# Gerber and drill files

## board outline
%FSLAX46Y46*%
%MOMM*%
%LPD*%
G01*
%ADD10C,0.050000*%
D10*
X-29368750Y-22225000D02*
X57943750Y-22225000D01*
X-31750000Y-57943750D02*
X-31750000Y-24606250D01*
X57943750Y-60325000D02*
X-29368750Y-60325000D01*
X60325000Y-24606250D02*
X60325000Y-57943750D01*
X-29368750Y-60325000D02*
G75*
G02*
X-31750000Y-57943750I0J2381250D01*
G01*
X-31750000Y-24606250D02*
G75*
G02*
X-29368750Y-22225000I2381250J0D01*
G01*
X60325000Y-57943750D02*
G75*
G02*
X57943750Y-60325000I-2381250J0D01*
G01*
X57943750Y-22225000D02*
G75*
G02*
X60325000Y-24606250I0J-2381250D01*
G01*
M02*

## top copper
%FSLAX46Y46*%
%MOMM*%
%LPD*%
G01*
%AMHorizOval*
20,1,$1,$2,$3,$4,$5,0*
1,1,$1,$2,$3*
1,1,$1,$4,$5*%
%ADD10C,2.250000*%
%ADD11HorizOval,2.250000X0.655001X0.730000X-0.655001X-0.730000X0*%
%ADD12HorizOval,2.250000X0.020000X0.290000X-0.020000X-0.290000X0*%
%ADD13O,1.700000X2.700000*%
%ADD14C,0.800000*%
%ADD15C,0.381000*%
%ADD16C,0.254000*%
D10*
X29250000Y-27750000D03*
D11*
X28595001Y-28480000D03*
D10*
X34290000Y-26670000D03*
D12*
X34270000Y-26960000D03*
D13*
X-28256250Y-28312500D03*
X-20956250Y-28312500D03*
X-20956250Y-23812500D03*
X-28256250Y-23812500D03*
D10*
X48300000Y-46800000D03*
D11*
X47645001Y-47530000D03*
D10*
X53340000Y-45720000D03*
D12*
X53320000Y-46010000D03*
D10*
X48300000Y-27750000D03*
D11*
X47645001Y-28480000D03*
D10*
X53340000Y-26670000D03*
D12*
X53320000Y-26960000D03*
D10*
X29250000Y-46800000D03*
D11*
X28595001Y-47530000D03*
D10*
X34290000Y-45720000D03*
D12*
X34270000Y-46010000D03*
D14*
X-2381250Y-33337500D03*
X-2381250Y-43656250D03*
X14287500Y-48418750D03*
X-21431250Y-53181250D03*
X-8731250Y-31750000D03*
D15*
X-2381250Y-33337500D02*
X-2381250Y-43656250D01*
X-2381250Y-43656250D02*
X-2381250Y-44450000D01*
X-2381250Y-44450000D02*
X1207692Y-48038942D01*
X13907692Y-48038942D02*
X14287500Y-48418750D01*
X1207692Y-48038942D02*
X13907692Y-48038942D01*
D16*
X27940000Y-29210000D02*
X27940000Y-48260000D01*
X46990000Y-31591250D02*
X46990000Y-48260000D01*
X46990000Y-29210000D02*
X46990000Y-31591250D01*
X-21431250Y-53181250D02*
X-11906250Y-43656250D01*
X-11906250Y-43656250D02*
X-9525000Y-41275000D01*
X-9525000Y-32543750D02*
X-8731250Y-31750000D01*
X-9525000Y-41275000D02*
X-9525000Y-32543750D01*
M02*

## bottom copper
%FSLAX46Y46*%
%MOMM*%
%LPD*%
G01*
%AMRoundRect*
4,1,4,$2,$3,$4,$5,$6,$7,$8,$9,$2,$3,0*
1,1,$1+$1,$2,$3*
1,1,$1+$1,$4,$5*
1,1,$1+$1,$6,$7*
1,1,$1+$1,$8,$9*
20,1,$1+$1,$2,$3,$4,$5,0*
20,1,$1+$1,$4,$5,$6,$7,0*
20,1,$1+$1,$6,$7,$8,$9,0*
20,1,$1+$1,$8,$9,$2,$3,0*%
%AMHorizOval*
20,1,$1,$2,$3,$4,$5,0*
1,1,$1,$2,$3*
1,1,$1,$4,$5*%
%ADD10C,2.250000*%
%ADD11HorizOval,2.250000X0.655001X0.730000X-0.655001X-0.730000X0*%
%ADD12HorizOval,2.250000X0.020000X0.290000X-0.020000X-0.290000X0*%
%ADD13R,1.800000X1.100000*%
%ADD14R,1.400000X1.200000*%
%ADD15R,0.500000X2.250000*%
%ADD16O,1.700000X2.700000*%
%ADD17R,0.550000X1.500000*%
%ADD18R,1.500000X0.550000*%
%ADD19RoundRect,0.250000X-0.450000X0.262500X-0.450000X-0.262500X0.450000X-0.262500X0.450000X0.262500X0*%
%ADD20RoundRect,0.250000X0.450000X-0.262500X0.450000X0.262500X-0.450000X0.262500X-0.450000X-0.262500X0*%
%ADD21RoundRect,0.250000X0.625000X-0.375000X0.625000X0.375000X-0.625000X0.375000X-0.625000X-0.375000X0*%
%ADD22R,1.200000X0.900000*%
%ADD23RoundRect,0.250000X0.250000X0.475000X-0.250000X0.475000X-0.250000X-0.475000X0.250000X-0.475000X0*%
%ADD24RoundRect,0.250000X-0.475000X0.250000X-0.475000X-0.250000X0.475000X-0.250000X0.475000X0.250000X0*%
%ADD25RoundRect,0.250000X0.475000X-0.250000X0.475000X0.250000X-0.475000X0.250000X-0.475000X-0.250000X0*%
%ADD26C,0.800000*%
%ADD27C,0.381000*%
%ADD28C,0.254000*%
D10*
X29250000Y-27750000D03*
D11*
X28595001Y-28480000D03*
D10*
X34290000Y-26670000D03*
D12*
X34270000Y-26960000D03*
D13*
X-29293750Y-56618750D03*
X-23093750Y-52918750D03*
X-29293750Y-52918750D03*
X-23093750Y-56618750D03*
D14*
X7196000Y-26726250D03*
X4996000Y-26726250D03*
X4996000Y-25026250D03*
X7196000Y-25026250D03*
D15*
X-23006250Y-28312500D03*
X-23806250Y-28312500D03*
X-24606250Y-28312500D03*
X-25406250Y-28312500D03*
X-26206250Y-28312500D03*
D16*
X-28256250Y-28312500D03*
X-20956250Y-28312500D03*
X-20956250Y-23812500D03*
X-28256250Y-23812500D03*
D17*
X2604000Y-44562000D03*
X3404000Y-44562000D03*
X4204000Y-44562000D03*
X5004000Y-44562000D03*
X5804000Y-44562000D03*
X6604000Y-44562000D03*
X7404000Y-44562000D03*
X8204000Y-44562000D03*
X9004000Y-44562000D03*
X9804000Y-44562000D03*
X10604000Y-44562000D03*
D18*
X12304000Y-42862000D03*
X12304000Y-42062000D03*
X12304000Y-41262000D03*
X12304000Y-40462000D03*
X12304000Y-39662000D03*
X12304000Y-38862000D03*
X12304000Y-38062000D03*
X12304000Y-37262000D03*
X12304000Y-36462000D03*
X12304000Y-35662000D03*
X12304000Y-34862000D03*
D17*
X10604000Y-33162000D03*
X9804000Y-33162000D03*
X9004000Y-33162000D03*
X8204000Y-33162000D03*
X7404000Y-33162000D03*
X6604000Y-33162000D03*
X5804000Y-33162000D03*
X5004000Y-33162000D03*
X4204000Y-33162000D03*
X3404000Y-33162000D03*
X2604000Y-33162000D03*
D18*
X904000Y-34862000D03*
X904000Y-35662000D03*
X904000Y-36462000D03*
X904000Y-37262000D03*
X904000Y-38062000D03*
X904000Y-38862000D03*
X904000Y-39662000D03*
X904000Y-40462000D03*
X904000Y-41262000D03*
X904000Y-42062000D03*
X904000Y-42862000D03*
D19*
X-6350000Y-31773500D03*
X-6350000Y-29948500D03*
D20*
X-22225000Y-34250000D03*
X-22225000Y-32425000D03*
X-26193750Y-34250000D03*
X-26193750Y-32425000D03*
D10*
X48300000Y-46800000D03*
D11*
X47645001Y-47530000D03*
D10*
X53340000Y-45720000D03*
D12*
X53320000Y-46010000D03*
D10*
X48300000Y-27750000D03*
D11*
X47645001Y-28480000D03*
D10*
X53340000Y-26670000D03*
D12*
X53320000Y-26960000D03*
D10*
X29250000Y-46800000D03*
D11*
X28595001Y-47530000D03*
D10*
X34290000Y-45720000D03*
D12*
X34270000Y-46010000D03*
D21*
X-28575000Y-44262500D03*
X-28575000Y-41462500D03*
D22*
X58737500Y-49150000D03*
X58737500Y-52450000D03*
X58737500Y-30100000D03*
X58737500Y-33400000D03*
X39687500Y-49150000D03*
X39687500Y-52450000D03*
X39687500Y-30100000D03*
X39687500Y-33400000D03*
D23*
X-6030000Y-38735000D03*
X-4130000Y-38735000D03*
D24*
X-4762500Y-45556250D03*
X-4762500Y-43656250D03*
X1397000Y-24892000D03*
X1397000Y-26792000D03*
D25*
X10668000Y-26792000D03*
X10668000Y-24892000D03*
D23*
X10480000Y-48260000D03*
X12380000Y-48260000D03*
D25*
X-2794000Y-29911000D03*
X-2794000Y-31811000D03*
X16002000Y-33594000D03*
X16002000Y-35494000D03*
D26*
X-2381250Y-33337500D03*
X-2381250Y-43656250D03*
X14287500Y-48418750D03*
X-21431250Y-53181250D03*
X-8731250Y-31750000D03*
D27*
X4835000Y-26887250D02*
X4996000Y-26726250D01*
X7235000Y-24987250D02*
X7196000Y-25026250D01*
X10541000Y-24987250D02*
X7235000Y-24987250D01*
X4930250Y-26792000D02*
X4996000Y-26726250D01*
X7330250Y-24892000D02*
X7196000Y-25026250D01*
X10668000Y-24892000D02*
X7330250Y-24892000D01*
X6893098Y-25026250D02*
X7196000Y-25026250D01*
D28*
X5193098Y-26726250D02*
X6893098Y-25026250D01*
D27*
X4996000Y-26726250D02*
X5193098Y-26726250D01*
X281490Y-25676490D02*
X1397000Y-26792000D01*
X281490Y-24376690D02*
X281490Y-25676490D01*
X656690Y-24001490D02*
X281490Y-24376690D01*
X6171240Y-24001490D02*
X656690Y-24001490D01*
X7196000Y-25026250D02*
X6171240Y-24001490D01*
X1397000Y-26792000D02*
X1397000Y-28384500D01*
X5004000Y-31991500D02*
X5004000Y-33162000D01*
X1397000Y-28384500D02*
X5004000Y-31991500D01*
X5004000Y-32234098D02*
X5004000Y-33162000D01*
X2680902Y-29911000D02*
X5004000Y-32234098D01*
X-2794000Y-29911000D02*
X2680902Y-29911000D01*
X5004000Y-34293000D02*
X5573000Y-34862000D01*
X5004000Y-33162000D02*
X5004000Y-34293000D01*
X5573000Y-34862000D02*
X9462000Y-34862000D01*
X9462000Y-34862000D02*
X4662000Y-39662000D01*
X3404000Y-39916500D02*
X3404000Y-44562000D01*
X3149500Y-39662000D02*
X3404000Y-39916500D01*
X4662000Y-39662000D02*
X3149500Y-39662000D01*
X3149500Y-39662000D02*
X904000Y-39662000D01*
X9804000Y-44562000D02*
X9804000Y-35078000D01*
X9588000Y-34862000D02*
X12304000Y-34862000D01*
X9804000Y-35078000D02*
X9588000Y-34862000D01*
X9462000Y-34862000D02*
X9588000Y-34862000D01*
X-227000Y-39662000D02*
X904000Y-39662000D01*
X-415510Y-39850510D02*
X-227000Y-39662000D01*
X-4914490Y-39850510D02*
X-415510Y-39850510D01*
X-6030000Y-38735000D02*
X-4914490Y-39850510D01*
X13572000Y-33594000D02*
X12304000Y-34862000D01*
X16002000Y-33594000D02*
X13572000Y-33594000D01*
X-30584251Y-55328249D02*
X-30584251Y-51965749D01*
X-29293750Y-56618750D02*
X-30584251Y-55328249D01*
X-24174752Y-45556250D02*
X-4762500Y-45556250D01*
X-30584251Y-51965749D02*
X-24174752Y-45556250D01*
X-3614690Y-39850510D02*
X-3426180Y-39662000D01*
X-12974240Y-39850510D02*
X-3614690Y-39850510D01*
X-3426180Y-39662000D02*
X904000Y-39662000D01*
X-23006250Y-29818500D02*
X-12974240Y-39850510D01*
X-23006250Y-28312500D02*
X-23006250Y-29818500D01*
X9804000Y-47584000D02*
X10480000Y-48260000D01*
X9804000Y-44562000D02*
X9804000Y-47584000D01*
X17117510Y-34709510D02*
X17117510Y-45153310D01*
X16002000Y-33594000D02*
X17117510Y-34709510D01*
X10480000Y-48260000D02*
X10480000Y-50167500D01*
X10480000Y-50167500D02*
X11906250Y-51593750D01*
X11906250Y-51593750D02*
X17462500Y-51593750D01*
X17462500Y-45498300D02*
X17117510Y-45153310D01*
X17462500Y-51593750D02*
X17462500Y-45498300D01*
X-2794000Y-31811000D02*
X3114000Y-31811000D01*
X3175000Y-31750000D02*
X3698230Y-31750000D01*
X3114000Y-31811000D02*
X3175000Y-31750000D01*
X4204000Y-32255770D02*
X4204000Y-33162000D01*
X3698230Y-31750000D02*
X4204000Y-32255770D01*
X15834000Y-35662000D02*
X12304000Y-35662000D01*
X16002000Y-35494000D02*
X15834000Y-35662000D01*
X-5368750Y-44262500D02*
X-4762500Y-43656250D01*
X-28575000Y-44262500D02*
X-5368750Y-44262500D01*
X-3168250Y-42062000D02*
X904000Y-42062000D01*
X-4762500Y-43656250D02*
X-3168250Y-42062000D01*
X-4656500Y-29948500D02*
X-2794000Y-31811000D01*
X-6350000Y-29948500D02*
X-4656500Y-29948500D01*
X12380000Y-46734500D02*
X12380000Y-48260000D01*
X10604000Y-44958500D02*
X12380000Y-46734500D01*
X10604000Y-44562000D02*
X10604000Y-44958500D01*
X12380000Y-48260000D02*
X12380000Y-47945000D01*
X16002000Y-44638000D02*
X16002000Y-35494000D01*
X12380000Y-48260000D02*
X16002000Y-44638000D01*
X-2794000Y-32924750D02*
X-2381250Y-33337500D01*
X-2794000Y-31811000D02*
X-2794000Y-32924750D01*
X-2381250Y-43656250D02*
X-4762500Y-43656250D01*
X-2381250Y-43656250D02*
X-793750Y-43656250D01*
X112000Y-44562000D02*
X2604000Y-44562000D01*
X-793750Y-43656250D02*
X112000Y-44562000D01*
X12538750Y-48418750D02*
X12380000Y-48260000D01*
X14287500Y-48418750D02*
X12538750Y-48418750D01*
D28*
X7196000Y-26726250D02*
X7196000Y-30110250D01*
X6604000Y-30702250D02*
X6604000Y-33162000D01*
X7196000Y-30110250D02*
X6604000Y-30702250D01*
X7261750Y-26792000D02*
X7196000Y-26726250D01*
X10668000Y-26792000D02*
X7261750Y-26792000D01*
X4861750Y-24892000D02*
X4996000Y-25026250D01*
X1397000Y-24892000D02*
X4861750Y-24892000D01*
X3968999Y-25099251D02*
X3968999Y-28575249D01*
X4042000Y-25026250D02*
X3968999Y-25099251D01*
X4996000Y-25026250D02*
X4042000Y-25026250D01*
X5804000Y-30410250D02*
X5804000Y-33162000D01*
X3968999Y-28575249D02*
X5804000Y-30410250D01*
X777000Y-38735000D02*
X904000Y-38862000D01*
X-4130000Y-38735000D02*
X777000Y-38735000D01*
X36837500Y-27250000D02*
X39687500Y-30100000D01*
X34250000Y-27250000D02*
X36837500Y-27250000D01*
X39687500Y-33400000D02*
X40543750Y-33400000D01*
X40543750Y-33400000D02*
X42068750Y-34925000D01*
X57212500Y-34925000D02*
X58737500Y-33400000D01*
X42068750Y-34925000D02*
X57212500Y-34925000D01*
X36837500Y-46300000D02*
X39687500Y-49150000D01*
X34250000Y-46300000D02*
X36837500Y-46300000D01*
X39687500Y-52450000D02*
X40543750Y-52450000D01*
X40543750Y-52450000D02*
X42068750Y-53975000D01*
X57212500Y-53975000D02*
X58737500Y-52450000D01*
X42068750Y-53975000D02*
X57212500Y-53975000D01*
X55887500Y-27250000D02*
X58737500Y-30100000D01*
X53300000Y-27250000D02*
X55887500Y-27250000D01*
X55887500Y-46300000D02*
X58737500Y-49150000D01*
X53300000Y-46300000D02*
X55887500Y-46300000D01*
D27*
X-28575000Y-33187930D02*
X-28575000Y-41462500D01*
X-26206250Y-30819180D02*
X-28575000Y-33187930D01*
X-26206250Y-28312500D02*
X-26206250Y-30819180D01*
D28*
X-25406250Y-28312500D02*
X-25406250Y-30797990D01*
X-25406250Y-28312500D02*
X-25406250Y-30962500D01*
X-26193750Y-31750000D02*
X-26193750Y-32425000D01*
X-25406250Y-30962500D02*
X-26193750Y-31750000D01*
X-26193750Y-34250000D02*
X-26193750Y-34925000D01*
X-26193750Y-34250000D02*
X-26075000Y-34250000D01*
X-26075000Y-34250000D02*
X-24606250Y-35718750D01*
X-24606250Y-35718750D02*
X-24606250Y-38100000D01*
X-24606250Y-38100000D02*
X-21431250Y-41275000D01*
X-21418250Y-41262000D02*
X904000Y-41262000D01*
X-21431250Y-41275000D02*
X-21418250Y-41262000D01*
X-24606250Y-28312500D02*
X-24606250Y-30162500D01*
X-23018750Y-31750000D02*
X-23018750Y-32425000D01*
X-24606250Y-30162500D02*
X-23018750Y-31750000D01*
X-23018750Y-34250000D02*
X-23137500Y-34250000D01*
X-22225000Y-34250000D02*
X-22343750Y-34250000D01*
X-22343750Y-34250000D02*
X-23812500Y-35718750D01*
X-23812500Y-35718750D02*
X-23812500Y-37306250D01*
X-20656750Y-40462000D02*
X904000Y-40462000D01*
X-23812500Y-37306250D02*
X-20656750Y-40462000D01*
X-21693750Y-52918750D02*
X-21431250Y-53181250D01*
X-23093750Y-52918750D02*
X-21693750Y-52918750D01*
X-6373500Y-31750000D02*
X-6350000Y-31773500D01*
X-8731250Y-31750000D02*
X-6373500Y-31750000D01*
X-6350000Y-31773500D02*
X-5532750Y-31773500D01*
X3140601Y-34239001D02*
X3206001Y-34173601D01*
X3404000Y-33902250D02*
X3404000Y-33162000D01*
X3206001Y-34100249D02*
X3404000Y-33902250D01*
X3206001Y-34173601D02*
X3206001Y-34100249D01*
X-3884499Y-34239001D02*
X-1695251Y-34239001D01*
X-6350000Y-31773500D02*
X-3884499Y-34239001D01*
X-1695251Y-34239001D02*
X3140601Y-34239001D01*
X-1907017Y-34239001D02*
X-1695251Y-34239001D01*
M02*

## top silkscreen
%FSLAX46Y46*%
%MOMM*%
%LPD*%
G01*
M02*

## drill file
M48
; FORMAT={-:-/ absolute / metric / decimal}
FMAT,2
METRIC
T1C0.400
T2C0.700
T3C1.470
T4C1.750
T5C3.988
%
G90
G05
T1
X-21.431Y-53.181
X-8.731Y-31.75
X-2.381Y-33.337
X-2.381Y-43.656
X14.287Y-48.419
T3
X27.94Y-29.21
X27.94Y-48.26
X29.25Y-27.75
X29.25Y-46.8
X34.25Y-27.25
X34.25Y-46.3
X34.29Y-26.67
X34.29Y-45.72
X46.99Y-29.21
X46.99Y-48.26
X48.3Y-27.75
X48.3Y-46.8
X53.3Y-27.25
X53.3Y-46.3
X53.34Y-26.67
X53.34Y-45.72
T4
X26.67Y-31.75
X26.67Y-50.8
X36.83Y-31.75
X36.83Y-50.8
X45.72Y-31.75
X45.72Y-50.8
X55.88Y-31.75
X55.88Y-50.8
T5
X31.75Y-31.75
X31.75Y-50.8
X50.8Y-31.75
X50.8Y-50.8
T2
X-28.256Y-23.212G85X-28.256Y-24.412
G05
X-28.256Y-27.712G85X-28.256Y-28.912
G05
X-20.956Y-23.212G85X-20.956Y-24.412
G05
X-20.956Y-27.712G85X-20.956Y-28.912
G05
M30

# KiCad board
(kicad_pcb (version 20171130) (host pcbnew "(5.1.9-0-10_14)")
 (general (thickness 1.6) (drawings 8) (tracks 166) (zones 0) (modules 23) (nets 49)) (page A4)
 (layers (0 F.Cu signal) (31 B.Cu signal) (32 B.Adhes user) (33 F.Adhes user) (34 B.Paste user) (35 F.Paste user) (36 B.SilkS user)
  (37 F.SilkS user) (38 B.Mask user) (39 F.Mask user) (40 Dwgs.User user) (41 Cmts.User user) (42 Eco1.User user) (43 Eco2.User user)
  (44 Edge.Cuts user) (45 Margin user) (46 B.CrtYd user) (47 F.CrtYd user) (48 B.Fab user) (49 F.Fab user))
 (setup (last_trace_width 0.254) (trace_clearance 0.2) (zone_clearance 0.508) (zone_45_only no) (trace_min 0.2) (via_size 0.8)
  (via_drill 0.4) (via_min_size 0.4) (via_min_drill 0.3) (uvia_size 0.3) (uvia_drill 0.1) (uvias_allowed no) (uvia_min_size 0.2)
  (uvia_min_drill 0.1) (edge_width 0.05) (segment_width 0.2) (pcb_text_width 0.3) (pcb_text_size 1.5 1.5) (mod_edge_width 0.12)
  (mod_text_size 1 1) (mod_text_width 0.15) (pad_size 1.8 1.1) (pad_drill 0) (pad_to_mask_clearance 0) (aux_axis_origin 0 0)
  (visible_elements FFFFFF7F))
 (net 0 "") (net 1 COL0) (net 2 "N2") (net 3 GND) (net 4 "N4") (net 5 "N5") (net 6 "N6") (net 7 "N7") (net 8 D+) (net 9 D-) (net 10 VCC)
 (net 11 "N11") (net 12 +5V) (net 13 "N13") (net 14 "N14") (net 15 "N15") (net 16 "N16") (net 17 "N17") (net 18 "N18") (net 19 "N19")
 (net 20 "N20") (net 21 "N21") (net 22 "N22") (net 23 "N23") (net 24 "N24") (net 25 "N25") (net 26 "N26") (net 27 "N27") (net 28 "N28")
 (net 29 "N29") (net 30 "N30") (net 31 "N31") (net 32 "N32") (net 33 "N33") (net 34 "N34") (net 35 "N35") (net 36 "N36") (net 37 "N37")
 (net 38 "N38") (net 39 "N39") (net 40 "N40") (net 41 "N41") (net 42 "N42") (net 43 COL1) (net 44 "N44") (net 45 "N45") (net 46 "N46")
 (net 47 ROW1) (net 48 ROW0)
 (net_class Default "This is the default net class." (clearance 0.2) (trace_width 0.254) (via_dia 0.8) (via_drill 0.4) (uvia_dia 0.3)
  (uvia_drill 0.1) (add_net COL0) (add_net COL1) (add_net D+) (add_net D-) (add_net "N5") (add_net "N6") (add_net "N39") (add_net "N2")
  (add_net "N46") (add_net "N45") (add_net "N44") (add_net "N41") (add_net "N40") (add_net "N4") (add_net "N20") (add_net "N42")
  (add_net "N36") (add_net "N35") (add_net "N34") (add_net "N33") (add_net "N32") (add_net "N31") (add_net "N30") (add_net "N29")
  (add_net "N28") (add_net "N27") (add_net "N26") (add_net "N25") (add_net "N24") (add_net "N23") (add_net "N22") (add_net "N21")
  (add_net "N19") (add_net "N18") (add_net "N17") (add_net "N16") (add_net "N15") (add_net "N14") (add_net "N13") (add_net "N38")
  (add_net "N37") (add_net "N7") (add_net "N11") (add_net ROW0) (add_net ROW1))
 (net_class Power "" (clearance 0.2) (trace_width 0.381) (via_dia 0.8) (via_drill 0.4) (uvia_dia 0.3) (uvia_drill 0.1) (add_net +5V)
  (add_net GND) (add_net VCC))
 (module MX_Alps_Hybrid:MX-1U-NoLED (layer F.Cu) (at 31.75 31.75)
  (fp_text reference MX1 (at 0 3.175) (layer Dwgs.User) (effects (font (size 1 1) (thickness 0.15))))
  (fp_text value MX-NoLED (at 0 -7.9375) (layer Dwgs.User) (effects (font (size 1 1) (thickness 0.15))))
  (pad "" np_thru_hole circle (at 5.08 0 48.0996) (size 1.75 1.75) (drill 1.75) (layers *.Cu *.Mask))
  (pad "" np_thru_hole circle (at -5.08 0 48.0996) (size 1.75 1.75) (drill 1.75) (layers *.Cu *.Mask))
  (pad 1 thru_hole circle (at -2.5 -4) (size 2.25 2.25) (drill 1.47) (layers *.Cu B.Mask) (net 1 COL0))
  (pad "" np_thru_hole circle (at 0 0) (size 3.9878 3.9878) (drill 3.9878) (layers *.Cu *.Mask))
  (pad 1 thru_hole oval (at -3.81 -2.54 48.0996) (size 4.211556 2.25) (drill 1.47 (offset 0.980778 0)) (layers *.Cu B.Mask) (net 1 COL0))
  (pad 2 thru_hole circle (at 2.54 -5.08) (size 2.25 2.25) (drill 1.47) (layers *.Cu B.Mask) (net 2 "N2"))
  (pad 2 thru_hole oval (at 2.5 -4.5 86.0548) (size 2.831378 2.25) (drill 1.47 (offset 0.290689 0)) (layers *.Cu B.Mask) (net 2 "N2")))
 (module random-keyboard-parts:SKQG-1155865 (layer B.Cu) (at -26.19375 54.76875 180)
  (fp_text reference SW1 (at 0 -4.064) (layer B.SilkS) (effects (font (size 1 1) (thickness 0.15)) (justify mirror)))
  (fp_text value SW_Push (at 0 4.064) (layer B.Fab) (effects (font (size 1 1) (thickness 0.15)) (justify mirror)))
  (pad 1 smd rect (at 3.1 -1.85 180) (size 1.8 1.1) (layers B.Cu B.Paste B.Mask) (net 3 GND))
  (pad 2 smd rect (at -3.1 1.85 180) (size 1.8 1.1) (layers B.Cu B.Paste B.Mask) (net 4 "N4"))
  (pad 3 smd rect (at 3.1 1.85 180) (size 1.8 1.1) (layers B.Cu B.Paste B.Mask))
  (pad 4 smd rect (at -3.1 -1.85 180) (size 1.8 1.1) (layers B.Cu B.Paste B.Mask)))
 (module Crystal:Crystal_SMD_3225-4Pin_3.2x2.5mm (layer B.Cu) (at 6.096 25.87625 180)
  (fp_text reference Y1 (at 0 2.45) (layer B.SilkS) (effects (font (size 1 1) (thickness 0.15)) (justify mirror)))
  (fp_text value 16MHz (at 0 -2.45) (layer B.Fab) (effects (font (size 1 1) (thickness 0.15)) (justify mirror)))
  (pad 1 smd rect (at -1.1 -0.85 180) (size 1.4 1.2) (layers B.Cu B.Paste B.Mask) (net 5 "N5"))
  (pad 2 smd rect (at 1.1 -0.85 180) (size 1.4 1.2) (layers B.Cu B.Paste B.Mask) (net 3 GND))
  (pad 3 smd rect (at 1.1 0.85 180) (size 1.4 1.2) (layers B.Cu B.Paste B.Mask) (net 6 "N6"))
  (pad 4 smd rect (at -1.1 0.85 180) (size 1.4 1.2) (layers B.Cu B.Paste B.Mask) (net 3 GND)))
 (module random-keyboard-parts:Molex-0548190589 (layer B.Cu) (at -24.60625 23.8125 270)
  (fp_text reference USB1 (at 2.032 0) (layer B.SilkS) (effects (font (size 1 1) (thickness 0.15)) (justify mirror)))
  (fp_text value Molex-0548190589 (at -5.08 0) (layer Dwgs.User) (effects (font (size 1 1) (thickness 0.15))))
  (pad 1 smd rect (at 4.5 -1.6 270) (size 2.25 0.5) (layers B.Cu B.Paste B.Mask) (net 3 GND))
  (pad 2 smd rect (at 4.5 -0.8 270) (size 2.25 0.5) (layers B.Cu B.Paste B.Mask) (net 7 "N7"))
  (pad 3 smd rect (at 4.5 0 270) (size 2.25 0.5) (layers B.Cu B.Paste B.Mask) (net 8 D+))
  (pad 4 smd rect (at 4.5 0.8 270) (size 2.25 0.5) (layers B.Cu B.Paste B.Mask) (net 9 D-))
  (pad 5 smd rect (at 4.5 1.6 270) (size 2.25 0.5) (layers B.Cu B.Paste B.Mask) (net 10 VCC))
  (pad 6 thru_hole oval (at 4.5 3.65 270) (size 2.7 1.7) (drill oval 1.9 0.7) (layers *.Cu *.Mask) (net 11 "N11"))
  (pad 6 thru_hole oval (at 4.5 -3.65 270) (size 2.7 1.7) (drill oval 1.9 0.7) (layers *.Cu *.Mask) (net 11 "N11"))
  (pad 6 thru_hole oval (at 0 -3.65 270) (size 2.7 1.7) (drill oval 1.9 0.7) (layers *.Cu *.Mask) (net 11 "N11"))
  (pad 6 thru_hole oval (at 0 3.65 270) (size 2.7 1.7) (drill oval 1.9 0.7) (layers *.Cu *.Mask) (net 11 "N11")))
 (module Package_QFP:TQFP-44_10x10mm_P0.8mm (layer B.Cu) (at 6.604 38.862)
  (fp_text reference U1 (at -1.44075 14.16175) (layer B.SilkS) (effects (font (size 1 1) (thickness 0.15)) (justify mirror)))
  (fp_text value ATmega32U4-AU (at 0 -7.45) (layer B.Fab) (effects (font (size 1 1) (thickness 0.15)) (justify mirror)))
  (pad 44 smd rect (at -4 5.7 270) (size 1.5 0.55) (layers B.Cu B.Paste B.Mask) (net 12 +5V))
  (pad 43 smd rect (at -3.2 5.7 270) (size 1.5 0.55) (layers B.Cu B.Paste B.Mask) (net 3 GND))
  (pad 42 smd rect (at -2.4 5.7 270) (size 1.5 0.55) (layers B.Cu B.Paste B.Mask) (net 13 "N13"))
  (pad 41 smd rect (at -1.6 5.7 270) (size 1.5 0.55) (layers B.Cu B.Paste B.Mask) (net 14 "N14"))
  (pad 40 smd rect (at -0.8 5.7 270) (size 1.5 0.55) (layers B.Cu B.Paste B.Mask) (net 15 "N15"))
  (pad 39 smd rect (at 0 5.7 270) (size 1.5 0.55) (layers B.Cu B.Paste B.Mask) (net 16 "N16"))
  (pad 38 smd rect (at 0.8 5.7 270) (size 1.5 0.55) (layers B.Cu B.Paste B.Mask) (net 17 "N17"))
  (pad 37 smd rect (at 1.6 5.7 270) (size 1.5 0.55) (layers B.Cu B.Paste B.Mask) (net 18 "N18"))
  (pad 36 smd rect (at 2.4 5.7 270) (size 1.5 0.55) (layers B.Cu B.Paste B.Mask) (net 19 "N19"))
  (pad 35 smd rect (at 3.2 5.7 270) (size 1.5 0.55) (layers B.Cu B.Paste B.Mask) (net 3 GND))
  (pad 34 smd rect (at 4 5.7 270) (size 1.5 0.55) (layers B.Cu B.Paste B.Mask) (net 12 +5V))
  (pad 33 smd rect (at 5.7 4) (size 1.5 0.55) (layers B.Cu B.Paste B.Mask) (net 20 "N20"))
  (pad 32 smd rect (at 5.7 3.2) (size 1.5 0.55) (layers B.Cu B.Paste B.Mask) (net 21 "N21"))
  (pad 31 smd rect (at 5.7 2.4) (size 1.5 0.55) (layers B.Cu B.Paste B.Mask) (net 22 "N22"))
  (pad 30 smd rect (at 5.7 1.6) (size 1.5 0.55) (layers B.Cu B.Paste B.Mask) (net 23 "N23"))
  (pad 29 smd rect (at 5.7 0.8) (size 1.5 0.55) (layers B.Cu B.Paste B.Mask) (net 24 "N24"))
  (pad 28 smd rect (at 5.7 0) (size 1.5 0.55) (layers B.Cu B.Paste B.Mask) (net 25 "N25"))
  (pad 27 smd rect (at 5.7 -0.8) (size 1.5 0.55) (layers B.Cu B.Paste B.Mask) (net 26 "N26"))
  (pad 26 smd rect (at 5.7 -1.6) (size 1.5 0.55) (layers B.Cu B.Paste B.Mask) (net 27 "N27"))
  (pad 25 smd rect (at 5.7 -2.4) (size 1.5 0.55) (layers B.Cu B.Paste B.Mask) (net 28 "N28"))
  (pad 24 smd rect (at 5.7 -3.2) (size 1.5 0.55) (layers B.Cu B.Paste B.Mask) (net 12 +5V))
  (pad 23 smd rect (at 5.7 -4) (size 1.5 0.55) (layers B.Cu B.Paste B.Mask) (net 3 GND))
  (pad 22 smd rect (at 4 -5.7 270) (size 1.5 0.55) (layers B.Cu B.Paste B.Mask) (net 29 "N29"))
  (pad 21 smd rect (at 3.2 -5.7 270) (size 1.5 0.55) (layers B.Cu B.Paste B.Mask) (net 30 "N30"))
  (pad 20 smd rect (at 2.4 -5.7 270) (size 1.5 0.55) (layers B.Cu B.Paste B.Mask) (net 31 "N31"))
  (pad 19 smd rect (at 1.6 -5.7 270) (size 1.5 0.55) (layers B.Cu B.Paste B.Mask) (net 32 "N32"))
  (pad 18 smd rect (at 0.8 -5.7 270) (size 1.5 0.55) (layers B.Cu B.Paste B.Mask) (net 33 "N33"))
  (pad 17 smd rect (at 0 -5.7 270) (size 1.5 0.55) (layers B.Cu B.Paste B.Mask) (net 5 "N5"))
  (pad 16 smd rect (at -0.8 -5.7 270) (size 1.5 0.55) (layers B.Cu B.Paste B.Mask) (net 6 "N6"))
  (pad 15 smd rect (at -1.6 -5.7 270) (size 1.5 0.55) (layers B.Cu B.Paste B.Mask) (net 3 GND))
  (pad 14 smd rect (at -2.4 -5.7 270) (size 1.5 0.55) (layers B.Cu B.Paste B.Mask) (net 12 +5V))
  (pad 13 smd rect (at -3.2 -5.7 270) (size 1.5 0.55) (layers B.Cu B.Paste B.Mask) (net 4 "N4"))
  (pad 12 smd rect (at -4 -5.7 270) (size 1.5 0.55) (layers B.Cu B.Paste B.Mask) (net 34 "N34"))
  (pad 11 smd rect (at -5.7 -4) (size 1.5 0.55) (layers B.Cu B.Paste B.Mask) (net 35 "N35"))
  (pad 10 smd rect (at -5.7 -3.2) (size 1.5 0.55) (layers B.Cu B.Paste B.Mask) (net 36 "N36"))
  (pad 9 smd rect (at -5.7 -2.4) (size 1.5 0.55) (layers B.Cu B.Paste B.Mask) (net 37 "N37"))
  (pad 8 smd rect (at -5.7 -1.6) (size 1.5 0.55) (layers B.Cu B.Paste B.Mask) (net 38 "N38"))
  (pad 7 smd rect (at -5.7 -0.8) (size 1.5 0.55) (layers B.Cu B.Paste B.Mask) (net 12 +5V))
  (pad 6 smd rect (at -5.7 0) (size 1.5 0.55) (layers B.Cu B.Paste B.Mask) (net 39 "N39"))
  (pad 5 smd rect (at -5.7 0.8) (size 1.5 0.55) (layers B.Cu B.Paste B.Mask) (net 3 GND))
  (pad 4 smd rect (at -5.7 1.6) (size 1.5 0.55) (layers B.Cu B.Paste B.Mask) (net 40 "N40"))
  (pad 3 smd rect (at -5.7 2.4) (size 1.5 0.55) (layers B.Cu B.Paste B.Mask) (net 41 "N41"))
  (pad 2 smd rect (at -5.7 3.2) (size 1.5 0.55) (layers B.Cu B.Paste B.Mask) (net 12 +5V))
  (pad 1 smd rect (at -5.7 4) (size 1.5 0.55) (layers B.Cu B.Paste B.Mask) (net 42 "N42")))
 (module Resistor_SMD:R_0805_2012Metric (layer B.Cu) (at -6.35 30.861 270)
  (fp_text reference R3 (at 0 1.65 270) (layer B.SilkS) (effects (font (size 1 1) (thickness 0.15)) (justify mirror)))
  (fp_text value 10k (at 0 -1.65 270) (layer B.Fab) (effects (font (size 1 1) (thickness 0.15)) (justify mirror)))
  (pad 2 smd roundrect (at 0.9125 0 270) (size 1.025 1.4) (layers B.Cu B.Paste B.Mask) (roundrect_rratio 0.243902) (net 4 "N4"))
  (pad 1 smd roundrect (at -0.9125 0 270) (size 1.025 1.4) (layers B.Cu B.Paste B.Mask) (roundrect_rratio 0.243902) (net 12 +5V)))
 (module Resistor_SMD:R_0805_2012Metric (layer B.Cu) (at -22.225 33.3375 90)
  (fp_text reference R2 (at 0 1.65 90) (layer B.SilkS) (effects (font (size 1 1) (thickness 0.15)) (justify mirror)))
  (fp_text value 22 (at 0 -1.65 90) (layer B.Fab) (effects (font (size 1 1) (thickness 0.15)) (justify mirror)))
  (pad 1 smd roundrect (at -0.9125 0 90) (size 1.025 1.4) (layers B.Cu B.Paste B.Mask) (roundrect_rratio 0.243902) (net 40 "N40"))
  (pad 2 smd roundrect (at 0.9125 0 90) (size 1.025 1.4) (layers B.Cu B.Paste B.Mask) (roundrect_rratio 0.243902) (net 8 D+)))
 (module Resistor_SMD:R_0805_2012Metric (layer B.Cu) (at -26.19375 33.3375 90)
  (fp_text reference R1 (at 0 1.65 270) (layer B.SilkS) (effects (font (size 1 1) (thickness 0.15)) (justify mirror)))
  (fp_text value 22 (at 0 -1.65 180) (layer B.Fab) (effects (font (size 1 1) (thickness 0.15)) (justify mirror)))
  (pad 1 smd roundrect (at -0.9125 0 90) (size 1.025 1.4) (layers B.Cu B.Paste B.Mask) (roundrect_rratio 0.243902) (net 41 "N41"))
  (pad 2 smd roundrect (at 0.9125 0 90) (size 1.025 1.4) (layers B.Cu B.Paste B.Mask) (roundrect_rratio 0.243902) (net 9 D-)))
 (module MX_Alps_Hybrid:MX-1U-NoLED (layer F.Cu) (at 50.8 50.8)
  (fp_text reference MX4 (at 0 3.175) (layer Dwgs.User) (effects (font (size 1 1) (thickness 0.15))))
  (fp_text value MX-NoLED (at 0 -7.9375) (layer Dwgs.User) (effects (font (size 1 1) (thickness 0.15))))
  (pad "" np_thru_hole circle (at 5.08 0 48.0996) (size 1.75 1.75) (drill 1.75) (layers *.Cu *.Mask))
  (pad "" np_thru_hole circle (at -5.08 0 48.0996) (size 1.75 1.75) (drill 1.75) (layers *.Cu *.Mask))
  (pad 1 thru_hole circle (at -2.5 -4) (size 2.25 2.25) (drill 1.47) (layers *.Cu B.Mask) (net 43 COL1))
  (pad "" np_thru_hole circle (at 0 0) (size 3.9878 3.9878) (drill 3.9878) (layers *.Cu *.Mask))
  (pad 1 thru_hole oval (at -3.81 -2.54 48.0996) (size 4.211556 2.25) (drill 1.47 (offset 0.980778 0)) (layers *.Cu B.Mask) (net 43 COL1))
  (pad 2 thru_hole circle (at 2.54 -5.08) (size 2.25 2.25) (drill 1.47) (layers *.Cu B.Mask) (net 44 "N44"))
  (pad 2 thru_hole oval (at 2.5 -4.5 86.0548) (size 2.831378 2.25) (drill 1.47 (offset 0.290689 0)) (layers *.Cu B.Mask) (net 44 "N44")))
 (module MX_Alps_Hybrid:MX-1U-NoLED (layer F.Cu) (at 50.8 31.75)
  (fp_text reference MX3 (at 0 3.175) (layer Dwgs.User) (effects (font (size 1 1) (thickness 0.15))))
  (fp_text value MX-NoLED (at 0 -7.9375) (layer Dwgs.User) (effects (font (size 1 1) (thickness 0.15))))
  (pad "" np_thru_hole circle (at 5.08 0 48.0996) (size 1.75 1.75) (drill 1.75) (layers *.Cu *.Mask))
  (pad "" np_thru_hole circle (at -5.08 0 48.0996) (size 1.75 1.75) (drill 1.75) (layers *.Cu *.Mask))
  (pad 1 thru_hole circle (at -2.5 -4) (size 2.25 2.25) (drill 1.47) (layers *.Cu B.Mask) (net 43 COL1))
  (pad "" np_thru_hole circle (at 0 0) (size 3.9878 3.9878) (drill 3.9878) (layers *.Cu *.Mask))
  (pad 1 thru_hole oval (at -3.81 -2.54 48.0996) (size 4.211556 2.25) (drill 1.47 (offset 0.980778 0)) (layers *.Cu B.Mask) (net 43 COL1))
  (pad 2 thru_hole circle (at 2.54 -5.08) (size 2.25 2.25) (drill 1.47) (layers *.Cu B.Mask) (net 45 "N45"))
  (pad 2 thru_hole oval (at 2.5 -4.5 86.0548) (size 2.831378 2.25) (drill 1.47 (offset 0.290689 0)) (layers *.Cu B.Mask) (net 45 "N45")))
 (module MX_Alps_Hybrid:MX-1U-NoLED (layer F.Cu) (at 31.75 50.8)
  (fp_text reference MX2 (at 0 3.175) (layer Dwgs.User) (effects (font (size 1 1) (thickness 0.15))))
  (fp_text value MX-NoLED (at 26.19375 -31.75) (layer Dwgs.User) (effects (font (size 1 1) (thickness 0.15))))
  (pad "" np_thru_hole circle (at 5.08 0 48.0996) (size 1.75 1.75) (drill 1.75) (layers *.Cu *.Mask))
  (pad "" np_thru_hole circle (at -5.08 0 48.0996) (size 1.75 1.75) (drill 1.75) (layers *.Cu *.Mask))
  (pad 1 thru_hole circle (at -2.5 -4) (size 2.25 2.25) (drill 1.47) (layers *.Cu B.Mask) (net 1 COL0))
  (pad "" np_thru_hole circle (at 0 0) (size 3.9878 3.9878) (drill 3.9878) (layers *.Cu *.Mask))
  (pad 1 thru_hole oval (at -3.81 -2.54 48.0996) (size 4.211556 2.25) (drill 1.47 (offset 0.980778 0)) (layers *.Cu B.Mask) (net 1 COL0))
  (pad 2 thru_hole circle (at 2.54 -5.08) (size 2.25 2.25) (drill 1.47) (layers *.Cu B.Mask) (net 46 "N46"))
  (pad 2 thru_hole oval (at 2.5 -4.5 86.0548) (size 2.831378 2.25) (drill 1.47 (offset 0.290689 0)) (layers *.Cu B.Mask) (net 46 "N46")))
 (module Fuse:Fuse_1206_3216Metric (layer B.Cu) (at -28.575 42.8625 90)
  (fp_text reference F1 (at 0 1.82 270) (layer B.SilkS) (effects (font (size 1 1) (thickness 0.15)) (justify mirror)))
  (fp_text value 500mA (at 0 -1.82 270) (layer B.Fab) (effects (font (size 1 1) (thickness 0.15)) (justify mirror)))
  (pad 1 smd roundrect (at -1.4 0 90) (size 1.25 1.75) (layers B.Cu B.Paste B.Mask) (roundrect_rratio 0.2) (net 12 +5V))
  (pad 2 smd roundrect (at 1.4 0 90) (size 1.25 1.75) (layers B.Cu B.Paste B.Mask) (roundrect_rratio 0.2) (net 10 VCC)))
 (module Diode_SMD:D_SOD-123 (layer B.Cu) (at 58.7375 50.8 90)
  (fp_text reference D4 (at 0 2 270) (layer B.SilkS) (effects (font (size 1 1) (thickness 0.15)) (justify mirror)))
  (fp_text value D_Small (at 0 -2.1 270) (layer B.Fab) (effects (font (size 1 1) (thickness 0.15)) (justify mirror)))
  (pad 2 smd rect (at 1.65 0 90) (size 0.9 1.2) (layers B.Cu B.Paste B.Mask) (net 44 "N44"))
  (pad 1 smd rect (at -1.65 0 90) (size 0.9 1.2) (layers B.Cu B.Paste B.Mask) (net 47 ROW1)))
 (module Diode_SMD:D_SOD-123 (layer B.Cu) (at 58.7375 31.75 90)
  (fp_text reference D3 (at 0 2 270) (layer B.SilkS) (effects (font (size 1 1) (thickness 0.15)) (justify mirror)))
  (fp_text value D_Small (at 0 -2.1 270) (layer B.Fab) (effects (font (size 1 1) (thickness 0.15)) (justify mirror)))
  (pad 2 smd rect (at 1.65 0 90) (size 0.9 1.2) (layers B.Cu B.Paste B.Mask) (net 45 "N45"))
  (pad 1 smd rect (at -1.65 0 90) (size 0.9 1.2) (layers B.Cu B.Paste B.Mask) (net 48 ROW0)))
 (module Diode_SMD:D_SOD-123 (layer B.Cu) (at 39.6875 50.8 90)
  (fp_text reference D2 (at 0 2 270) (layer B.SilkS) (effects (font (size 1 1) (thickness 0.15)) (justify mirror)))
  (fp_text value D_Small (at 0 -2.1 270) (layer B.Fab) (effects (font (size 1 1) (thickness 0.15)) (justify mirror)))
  (pad 2 smd rect (at 1.65 0 90) (size 0.9 1.2) (layers B.Cu B.Paste B.Mask) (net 46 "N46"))
  (pad 1 smd rect (at -1.65 0 90) (size 0.9 1.2) (layers B.Cu B.Paste B.Mask) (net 47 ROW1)))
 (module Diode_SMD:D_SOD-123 (layer B.Cu) (at 39.6875 31.75 90)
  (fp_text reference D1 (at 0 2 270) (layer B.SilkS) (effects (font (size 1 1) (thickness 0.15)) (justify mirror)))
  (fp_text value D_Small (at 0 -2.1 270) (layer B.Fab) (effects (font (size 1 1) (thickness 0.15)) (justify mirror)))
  (pad 2 smd rect (at 1.65 0 90) (size 0.9 1.2) (layers B.Cu B.Paste B.Mask) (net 2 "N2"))
  (pad 1 smd rect (at -1.65 0 90) (size 0.9 1.2) (layers B.Cu B.Paste B.Mask) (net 48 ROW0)))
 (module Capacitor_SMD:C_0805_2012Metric (layer B.Cu) (at -5.08 38.735 180)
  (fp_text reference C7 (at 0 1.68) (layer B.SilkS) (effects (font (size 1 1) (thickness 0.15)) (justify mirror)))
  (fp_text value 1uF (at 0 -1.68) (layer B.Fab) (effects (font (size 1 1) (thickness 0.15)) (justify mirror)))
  (pad 2 smd roundrect (at 0.95 0 180) (size 1 1.45) (layers B.Cu B.Paste B.Mask) (roundrect_rratio 0.25) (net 3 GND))
  (pad 1 smd roundrect (at -0.95 0 180) (size 1 1.45) (layers B.Cu B.Paste B.Mask) (roundrect_rratio 0.25) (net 39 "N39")))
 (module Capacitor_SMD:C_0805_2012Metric (layer B.Cu) (at -4.7625 44.60625 270)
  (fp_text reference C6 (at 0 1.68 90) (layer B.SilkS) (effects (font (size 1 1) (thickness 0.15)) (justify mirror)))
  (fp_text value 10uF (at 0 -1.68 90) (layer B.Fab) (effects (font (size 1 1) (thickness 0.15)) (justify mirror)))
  (pad 2 smd roundrect (at 0.95 0 270) (size 1 1.45) (layers B.Cu B.Paste B.Mask) (roundrect_rratio 0.25) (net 3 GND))
  (pad 1 smd roundrect (at -0.95 0 270) (size 1 1.45) (layers B.Cu B.Paste B.Mask) (roundrect_rratio 0.25) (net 12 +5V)))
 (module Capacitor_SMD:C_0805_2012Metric (layer B.Cu) (at 1.397 25.842 270)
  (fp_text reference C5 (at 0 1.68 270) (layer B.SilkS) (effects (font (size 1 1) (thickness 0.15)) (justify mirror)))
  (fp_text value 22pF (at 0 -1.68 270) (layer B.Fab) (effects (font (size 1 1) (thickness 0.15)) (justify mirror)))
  (pad 1 smd roundrect (at -0.95 0 270) (size 1 1.45) (layers B.Cu B.Paste B.Mask) (roundrect_rratio 0.25) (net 6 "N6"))
  (pad 2 smd roundrect (at 0.95 0 270) (size 1 1.45) (layers B.Cu B.Paste B.Mask) (roundrect_rratio 0.25) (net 3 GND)))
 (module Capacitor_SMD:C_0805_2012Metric (layer B.Cu) (at 10.668 25.842 90)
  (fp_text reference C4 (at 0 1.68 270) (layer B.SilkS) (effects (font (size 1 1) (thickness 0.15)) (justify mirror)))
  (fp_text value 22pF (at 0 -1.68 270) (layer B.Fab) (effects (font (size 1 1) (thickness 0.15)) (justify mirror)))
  (pad 1 smd roundrect (at -0.95 0 90) (size 1 1.45) (layers B.Cu B.Paste B.Mask) (roundrect_rratio 0.25) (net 5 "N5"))
  (pad 2 smd roundrect (at 0.95 0 90) (size 1 1.45) (layers B.Cu B.Paste B.Mask) (roundrect_rratio 0.25) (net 3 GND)))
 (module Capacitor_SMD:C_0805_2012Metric (layer B.Cu) (at 11.43 48.26 180)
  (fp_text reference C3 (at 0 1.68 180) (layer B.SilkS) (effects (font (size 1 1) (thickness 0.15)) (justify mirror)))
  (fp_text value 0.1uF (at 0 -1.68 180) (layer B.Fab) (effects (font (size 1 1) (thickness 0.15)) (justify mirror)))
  (pad 2 smd roundrect (at 0.95 0 180) (size 1 1.45) (layers B.Cu B.Paste B.Mask) (roundrect_rratio 0.25) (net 3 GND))
  (pad 1 smd roundrect (at -0.95 0 180) (size 1 1.45) (layers B.Cu B.Paste B.Mask) (roundrect_rratio 0.25) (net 12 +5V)))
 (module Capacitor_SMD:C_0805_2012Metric (layer B.Cu) (at -2.794 30.861 90)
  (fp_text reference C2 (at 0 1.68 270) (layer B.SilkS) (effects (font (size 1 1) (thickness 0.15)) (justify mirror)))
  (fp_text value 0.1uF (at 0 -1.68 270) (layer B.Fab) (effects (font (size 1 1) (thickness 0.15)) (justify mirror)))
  (pad 2 smd roundrect (at 0.95 0 90) (size 1 1.45) (layers B.Cu B.Paste B.Mask) (roundrect_rratio 0.25) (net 3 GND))
  (pad 1 smd roundrect (at -0.95 0 90) (size 1 1.45) (layers B.Cu B.Paste B.Mask) (roundrect_rratio 0.25) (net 12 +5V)))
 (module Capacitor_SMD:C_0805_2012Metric (layer B.Cu) (at 16.002 34.544 90)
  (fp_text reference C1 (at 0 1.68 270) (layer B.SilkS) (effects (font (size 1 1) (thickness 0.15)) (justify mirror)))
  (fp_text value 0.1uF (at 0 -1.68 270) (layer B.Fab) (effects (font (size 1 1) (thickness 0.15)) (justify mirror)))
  (pad 2 smd roundrect (at 0.95 0 90) (size 1 1.45) (layers B.Cu B.Paste B.Mask) (roundrect_rratio 0.25) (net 3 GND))
  (pad 1 smd roundrect (at -0.95 0 90) (size 1 1.45) (layers B.Cu B.Paste B.Mask) (roundrect_rratio 0.25) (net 12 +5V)))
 (gr_line (start -29.36875 22.225) (end 57.94375 22.225) (layer Edge.Cuts) (width 0.05))
 (gr_line (start -31.75 57.94375) (end -31.75 24.60625) (layer Edge.Cuts) (width 0.05))
 (gr_line (start 57.94375 60.325) (end -29.36875 60.325) (layer Edge.Cuts) (width 0.05))
 (gr_line (start 60.325 24.60625) (end 60.325 57.94375) (layer Edge.Cuts) (width 0.05))
 (gr_arc (start -29.36875 57.94375) (end -31.75 57.94375) (angle -90) (layer Edge.Cuts) (width 0.05))
 (gr_arc (start -29.36875 24.60625) (end -29.36875 22.225) (angle -90) (layer Edge.Cuts) (width 0.05))
 (gr_arc (start 57.94375 57.94375) (end 57.94375 60.325) (angle -90) (layer Edge.Cuts) (width 0.05))
 (gr_arc (start 57.94375 24.60625) (end 60.325 24.60625) (angle -90) (layer Edge.Cuts) (width 0.05))
 (segment (start 4.835 26.88725) (end 4.996 26.72625) (width 0.381) (layer B.Cu) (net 3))
 (segment (start 7.235 24.98725) (end 7.196 25.02625) (width 0.381) (layer B.Cu) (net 3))
 (segment (start 10.541 24.98725) (end 7.235 24.98725) (width 0.381) (layer B.Cu) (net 3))
 (segment (start 4.93025 26.792) (end 4.996 26.72625) (width 0.381) (layer B.Cu) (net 3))
 (segment (start 7.33025 24.892) (end 7.196 25.02625) (width 0.381) (layer B.Cu) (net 3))
 (segment (start 10.668 24.892) (end 7.33025 24.892) (width 0.381) (layer B.Cu) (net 3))
 (segment (start 6.893098 25.02625) (end 7.196 25.02625) (width 0.381) (layer B.Cu) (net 3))
 (segment (start 5.193098 26.72625) (end 6.893098 25.02625) (width 0.254) (layer B.Cu) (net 3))
 (segment (start 4.996 26.72625) (end 5.193098 26.72625) (width 0.381) (layer B.Cu) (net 3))
 (segment (start 0.28149 25.67649) (end 1.397 26.792) (width 0.381) (layer B.Cu) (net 3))
 (segment (start 0.28149 24.37669) (end 0.28149 25.67649) (width 0.381) (layer B.Cu) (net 3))
 (segment (start 0.65669 24.00149) (end 0.28149 24.37669) (width 0.381) (layer B.Cu) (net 3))
 (segment (start 6.17124 24.00149) (end 0.65669 24.00149) (width 0.381) (layer B.Cu) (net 3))
 (segment (start 7.196 25.02625) (end 6.17124 24.00149) (width 0.381) (layer B.Cu) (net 3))
 (segment (start 1.397 26.792) (end 1.397 28.3845) (width 0.381) (layer B.Cu) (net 3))
 (segment (start 5.004 31.9915) (end 5.004 33.162) (width 0.381) (layer B.Cu) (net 3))
 (segment (start 1.397 28.3845) (end 5.004 31.9915) (width 0.381) (layer B.Cu) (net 3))
 (segment (start 5.004 32.234098) (end 5.004 33.162) (width 0.381) (layer B.Cu) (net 3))
 (segment (start 2.680902 29.911) (end 5.004 32.234098) (width 0.381) (layer B.Cu) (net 3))
 (segment (start -2.794 29.911) (end 2.680902 29.911) (width 0.381) (layer B.Cu) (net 3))
 (segment (start 5.004 34.293) (end 5.573 34.862) (width 0.381) (layer B.Cu) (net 3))
 (segment (start 5.004 33.162) (end 5.004 34.293) (width 0.381) (layer B.Cu) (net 3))
 (segment (start 5.573 34.862) (end 9.462 34.862) (width 0.381) (layer B.Cu) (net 3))
 (segment (start 9.462 34.862) (end 4.662 39.662) (width 0.381) (layer B.Cu) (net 3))
 (segment (start 3.404 39.9165) (end 3.404 44.562) (width 0.381) (layer B.Cu) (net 3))
 (segment (start 3.1495 39.662) (end 3.404 39.9165) (width 0.381) (layer B.Cu) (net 3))
 (segment (start 4.662 39.662) (end 3.1495 39.662) (width 0.381) (layer B.Cu) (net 3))
 (segment (start 3.1495 39.662) (end 0.904 39.662) (width 0.381) (layer B.Cu) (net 3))
 (segment (start 9.804 44.562) (end 9.804 35.078) (width 0.381) (layer B.Cu) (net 3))
 (segment (start 9.588 34.862) (end 12.304 34.862) (width 0.381) (layer B.Cu) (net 3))
 (segment (start 9.804 35.078) (end 9.588 34.862) (width 0.381) (layer B.Cu) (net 3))
 (segment (start 9.462 34.862) (end 9.588 34.862) (width 0.381) (layer B.Cu) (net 3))
 (segment (start -0.227 39.662) (end 0.904 39.662) (width 0.381) (layer B.Cu) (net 3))
 (segment (start -0.41551 39.85051) (end -0.227 39.662) (width 0.381) (layer B.Cu) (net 3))
 (segment (start -4.91449 39.85051) (end -0.41551 39.85051) (width 0.381) (layer B.Cu) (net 3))
 (segment (start -6.03 38.735) (end -4.91449 39.85051) (width 0.381) (layer B.Cu) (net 3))
 (segment (start 13.572 33.594) (end 12.304 34.862) (width 0.381) (layer B.Cu) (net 3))
 (segment (start 16.002 33.594) (end 13.572 33.594) (width 0.381) (layer B.Cu) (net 3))
 (segment (start -30.584251 55.328249) (end -30.584251 51.965749) (width 0.381) (layer B.Cu) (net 3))
 (segment (start -29.29375 56.61875) (end -30.584251 55.328249) (width 0.381) (layer B.Cu) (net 3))
 (segment (start -24.174752 45.55625) (end -4.7625 45.55625) (width 0.381) (layer B.Cu) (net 3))
 (segment (start -30.584251 51.965749) (end -24.174752 45.55625) (width 0.381) (layer B.Cu) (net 3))
 (segment (start -3.61469 39.85051) (end -3.42618 39.662) (width 0.381) (layer B.Cu) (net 3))
 (segment (start -12.97424 39.85051) (end -3.61469 39.85051) (width 0.381) (layer B.Cu) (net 3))
 (segment (start -3.42618 39.662) (end 0.904 39.662) (width 0.381) (layer B.Cu) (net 3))
 (segment (start -23.00625 29.8185) (end -12.97424 39.85051) (width 0.381) (layer B.Cu) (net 3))
 (segment (start -23.00625 28.3125) (end -23.00625 29.8185) (width 0.381) (layer B.Cu) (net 3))
 (segment (start 9.804 47.584) (end 10.48 48.26) (width 0.381) (layer B.Cu) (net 3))
 (segment (start 9.804 44.562) (end 9.804 47.584) (width 0.381) (layer B.Cu) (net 3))
 (segment (start 17.11751 34.70951) (end 17.11751 45.15331) (width 0.381) (layer B.Cu) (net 3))
 (segment (start 16.002 33.594) (end 17.11751 34.70951) (width 0.381) (layer B.Cu) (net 3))
 (segment (start 10.48 48.26) (end 10.48 50.1675) (width 0.381) (layer B.Cu) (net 3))
 (segment (start 10.48 50.1675) (end 11.90625 51.59375) (width 0.381) (layer B.Cu) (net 3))
 (segment (start 11.90625 51.59375) (end 17.4625 51.59375) (width 0.381) (layer B.Cu) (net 3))
 (segment (start 17.4625 45.4983) (end 17.11751 45.15331) (width 0.381) (layer B.Cu) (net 3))
 (segment (start 17.4625 51.59375) (end 17.4625 45.4983) (width 0.381) (layer B.Cu) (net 3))
 (segment (start -2.794 31.811) (end 3.114 31.811) (width 0.381) (layer B.Cu) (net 12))
 (segment (start 3.175 31.75) (end 3.69823 31.75) (width 0.381) (layer B.Cu) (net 12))
 (segment (start 3.114 31.811) (end 3.175 31.75) (width 0.381) (layer B.Cu) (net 12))
 (segment (start 4.204 32.25577) (end 4.204 33.162) (width 0.381) (layer B.Cu) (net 12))
 (segment (start 3.69823 31.75) (end 4.204 32.25577) (width 0.381) (layer B.Cu) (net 12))
 (segment (start 15.834 35.662) (end 12.304 35.662) (width 0.381) (layer B.Cu) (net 12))
 (segment (start 16.002 35.494) (end 15.834 35.662) (width 0.381) (layer B.Cu) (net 12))
 (segment (start -5.36875 44.2625) (end -4.7625 43.65625) (width 0.381) (layer B.Cu) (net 12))
 (segment (start -28.575 44.2625) (end -5.36875 44.2625) (width 0.381) (layer B.Cu) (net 12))
 (segment (start -3.16825 42.062) (end 0.904 42.062) (width 0.381) (layer B.Cu) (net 12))
 (segment (start -4.7625 43.65625) (end -3.16825 42.062) (width 0.381) (layer B.Cu) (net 12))
 (segment (start -4.6565 29.9485) (end -2.794 31.811) (width 0.381) (layer B.Cu) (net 12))
 (segment (start -6.35 29.9485) (end -4.6565 29.9485) (width 0.381) (layer B.Cu) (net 12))
 (segment (start 12.38 46.7345) (end 12.38 48.26) (width 0.381) (layer B.Cu) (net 12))
 (segment (start 10.604 44.9585) (end 12.38 46.7345) (width 0.381) (layer B.Cu) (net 12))
 (segment (start 10.604 44.562) (end 10.604 44.9585) (width 0.381) (layer B.Cu) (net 12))
 (segment (start 12.38 48.26) (end 12.38 47.945) (width 0.381) (layer B.Cu) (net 12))
 (segment (start 16.002 44.638) (end 16.002 35.494) (width 0.381) (layer B.Cu) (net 12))
 (segment (start 12.38 48.26) (end 16.002 44.638) (width 0.381) (layer B.Cu) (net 12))
 (via (at -2.38125 33.3375) (size 0.8) (drill 0.4) (layers F.Cu B.Cu) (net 12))
 (segment (start -2.794 32.92475) (end -2.38125 33.3375) (width 0.381) (layer B.Cu) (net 12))
 (segment (start -2.794 31.811) (end -2.794 32.92475) (width 0.381) (layer B.Cu) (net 12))
 (via (at -2.38125 43.65625) (size 0.8) (drill 0.4) (layers F.Cu B.Cu) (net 12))
 (segment (start -2.38125 33.3375) (end -2.38125 43.65625) (width 0.381) (layer F.Cu) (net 12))
 (segment (start -2.38125 43.65625) (end -4.7625 43.65625) (width 0.381) (layer B.Cu) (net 12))
 (segment (start -2.38125 43.65625) (end -0.79375 43.65625) (width 0.381) (layer B.Cu) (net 12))
 (segment (start 0.112 44.562) (end 2.604 44.562) (width 0.381) (layer B.Cu) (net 12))
 (segment (start -0.79375 43.65625) (end 0.112 44.562) (width 0.381) (layer B.Cu) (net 12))
 (segment (start -2.38125 43.65625) (end -2.38125 44.45) (width 0.381) (layer F.Cu) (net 12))
 (segment (start -2.38125 44.45) (end 1.207692 48.038942) (width 0.381) (layer F.Cu) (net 12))
 (via (at 14.2875 48.41875) (size 0.8) (drill 0.4) (layers F.Cu B.Cu) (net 12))
 (segment (start 13.907692 48.038942) (end 14.2875 48.41875) (width 0.381) (layer F.Cu) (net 12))
 (segment (start 1.207692 48.038942) (end 13.907692 48.038942) (width 0.381) (layer F.Cu) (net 12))
 (segment (start 12.53875 48.41875) (end 12.38 48.26) (width 0.381) (layer B.Cu) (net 12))
 (segment (start 14.2875 48.41875) (end 12.53875 48.41875) (width 0.381) (layer B.Cu) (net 12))
 (segment (start 7.196 26.72625) (end 7.196 30.11025) (width 0.254) (layer B.Cu) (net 5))
 (segment (start 6.604 30.70225) (end 6.604 33.162) (width 0.254) (layer B.Cu) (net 5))
 (segment (start 7.196 30.11025) (end 6.604 30.70225) (width 0.254) (layer B.Cu) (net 5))
 (segment (start 7.26175 26.792) (end 7.196 26.72625) (width 0.254) (layer B.Cu) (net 5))
 (segment (start 10.668 26.792) (end 7.26175 26.792) (width 0.254) (layer B.Cu) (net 5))
 (segment (start 4.86175 24.892) (end 4.996 25.02625) (width 0.254) (layer B.Cu) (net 6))
 (segment (start 1.397 24.892) (end 4.86175 24.892) (width 0.254) (layer B.Cu) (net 6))
 (segment (start 3.968999 25.099251) (end 3.968999 28.575249) (width 0.254) (layer B.Cu) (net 6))
 (segment (start 4.042 25.02625) (end 3.968999 25.099251) (width 0.254) (layer B.Cu) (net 6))
 (segment (start 4.996 25.02625) (end 4.042 25.02625) (width 0.254) (layer B.Cu) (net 6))
 (segment (start 5.804 30.41025) (end 5.804 33.162) (width 0.254) (layer B.Cu) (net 6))
 (segment (start 3.968999 28.575249) (end 5.804 30.41025) (width 0.254) (layer B.Cu) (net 6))
 (segment (start 0.777 38.735) (end 0.904 38.862) (width 0.254) (layer B.Cu) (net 39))
 (segment (start -4.13 38.735) (end 0.777 38.735) (width 0.254) (layer B.Cu) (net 39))
 (segment (start 36.8375 27.25) (end 39.6875 30.1) (width 0.254) (layer B.Cu) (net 2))
 (segment (start 34.25 27.25) (end 36.8375 27.25) (width 0.254) (layer B.Cu) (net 2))
 (segment (start 39.6875 33.4) (end 40.54375 33.4) (width 0.254) (layer B.Cu) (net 48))
 (segment (start 40.54375 33.4) (end 42.06875 34.925) (width 0.254) (layer B.Cu) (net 48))
 (segment (start 57.2125 34.925) (end 58.7375 33.4) (width 0.254) (layer B.Cu) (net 48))
 (segment (start 42.06875 34.925) (end 57.2125 34.925) (width 0.254) (layer B.Cu) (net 48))
 (segment (start 36.8375 46.3) (end 39.6875 49.15) (width 0.254) (layer B.Cu) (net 46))
 (segment (start 34.25 46.3) (end 36.8375 46.3) (width 0.254) (layer B.Cu) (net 46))
 (segment (start 39.6875 52.45) (end 40.54375 52.45) (width 0.254) (layer B.Cu) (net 47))
 (segment (start 40.54375 52.45) (end 42.06875 53.975) (width 0.254) (layer B.Cu) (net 47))
 (segment (start 57.2125 53.975) (end 58.7375 52.45) (width 0.254) (layer B.Cu) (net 47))
 (segment (start 42.06875 53.975) (end 57.2125 53.975) (width 0.254) (layer B.Cu) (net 47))
 (segment (start 55.8875 27.25) (end 58.7375 30.1) (width 0.254) (layer B.Cu) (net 45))
 (segment (start 53.3 27.25) (end 55.8875 27.25) (width 0.254) (layer B.Cu) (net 45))
 (segment (start 55.8875 46.3) (end 58.7375 49.15) (width 0.254) (layer B.Cu) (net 44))
 (segment (start 53.3 46.3) (end 55.8875 46.3) (width 0.254) (layer B.Cu) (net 44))
 (segment (start -28.575 33.18793) (end -28.575 41.4625) (width 0.381) (layer B.Cu) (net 10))
 (segment (start -26.20625 30.81918) (end -28.575 33.18793) (width 0.381) (layer B.Cu) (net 10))
 (segment (start -26.20625 28.3125) (end -26.20625 30.81918) (width 0.381) (layer B.Cu) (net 10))
 (segment (start 27.94 29.21) (end 27.94 48.26) (width 0.254) (layer F.Cu) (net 1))
 (segment (start 46.99 31.59125) (end 46.99 48.26) (width 0.254) (layer F.Cu) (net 43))
 (segment (start 46.99 29.21) (end 46.99 31.59125) (width 0.254) (layer F.Cu) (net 43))
 (segment (start -25.40625 28.3125) (end -25.40625 30.79799) (width 0.254) (layer B.Cu) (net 9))
 (segment (start -25.40625 28.3125) (end -25.40625 30.9625) (width 0.254) (layer B.Cu) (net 9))
 (segment (start -26.19375 31.75) (end -26.19375 32.425) (width 0.254) (layer B.Cu) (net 9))
 (segment (start -25.40625 30.9625) (end -26.19375 31.75) (width 0.254) (layer B.Cu) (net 9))
 (segment (start -26.19375 34.25) (end -26.19375 34.925) (width 0.254) (layer B.Cu) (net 41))
 (segment (start -26.19375 34.25) (end -26.075 34.25) (width 0.254) (layer B.Cu) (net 41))
 (segment (start -26.075 34.25) (end -24.60625 35.71875) (width 0.254) (layer B.Cu) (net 41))
 (segment (start -24.60625 35.71875) (end -24.60625 38.1) (width 0.254) (layer B.Cu) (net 41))
 (segment (start -24.60625 38.1) (end -21.43125 41.275) (width 0.254) (layer B.Cu) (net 41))
 (segment (start -21.41825 41.262) (end 0.904 41.262) (width 0.254) (layer B.Cu) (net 41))
 (segment (start -21.43125 41.275) (end -21.41825 41.262) (width 0.254) (layer B.Cu) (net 41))
 (segment (start -24.60625 28.3125) (end -24.60625 30.1625) (width 0.254) (layer B.Cu) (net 8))
 (segment (start -23.01875 31.75) (end -23.01875 32.425) (width 0.254) (layer B.Cu) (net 8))
 (segment (start -24.60625 30.1625) (end -23.01875 31.75) (width 0.254) (layer B.Cu) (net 8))
 (segment (start -23.01875 34.25) (end -23.1375 34.25) (width 0.254) (layer B.Cu) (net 40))
 (segment (start -22.225 34.25) (end -22.34375 34.25) (width 0.254) (layer B.Cu) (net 40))
 (segment (start -22.34375 34.25) (end -23.8125 35.71875) (width 0.254) (layer B.Cu) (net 40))
 (segment (start -23.8125 35.71875) (end -23.8125 37.30625) (width 0.254) (layer B.Cu) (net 40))
 (segment (start -20.65675 40.462) (end 0.904 40.462) (width 0.254) (layer B.Cu) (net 40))
 (segment (start -23.8125 37.30625) (end -20.65675 40.462) (width 0.254) (layer B.Cu) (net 40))
 (via (at -21.43125 53.18125) (size 0.8) (drill 0.4) (layers F.Cu B.Cu) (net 4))
 (segment (start -21.69375 52.91875) (end -21.43125 53.18125) (width 0.254) (layer B.Cu) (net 4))
 (segment (start -23.09375 52.91875) (end -21.69375 52.91875) (width 0.254) (layer B.Cu) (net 4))
 (segment (start -21.43125 53.18125) (end -11.90625 43.65625) (width 0.254) (layer F.Cu) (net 4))
 (segment (start -11.90625 43.65625) (end -9.525 41.275) (width 0.254) (layer F.Cu) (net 4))
 (segment (start -9.525 32.54375) (end -8.73125 31.75) (width 0.254) (layer F.Cu) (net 4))
 (via (at -8.73125 31.75) (size 0.8) (drill 0.4) (layers F.Cu B.Cu) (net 4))
 (segment (start -9.525 41.275) (end -9.525 32.54375) (width 0.254) (layer F.Cu) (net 4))
 (segment (start -6.3735 31.75) (end -6.35 31.7735) (width 0.254) (layer B.Cu) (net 4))
 (segment (start -8.73125 31.75) (end -6.3735 31.75) (width 0.254) (layer B.Cu) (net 4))
 (segment (start -6.35 31.7735) (end -5.53275 31.7735) (width 0.254) (layer B.Cu) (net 4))
 (segment (start 3.140601 34.239001) (end 3.206001 34.173601) (width 0.254) (layer B.Cu) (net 4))
 (segment (start 3.404 33.90225) (end 3.404 33.162) (width 0.254) (layer B.Cu) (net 4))
 (segment (start 3.206001 34.100249) (end 3.404 33.90225) (width 0.254) (layer B.Cu) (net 4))
 (segment (start 3.206001 34.173601) (end 3.206001 34.100249) (width 0.254) (layer B.Cu) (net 4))
 (segment (start -3.884499 34.239001) (end -1.695251 34.239001) (width 0.254) (layer B.Cu) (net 4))
 (segment (start -6.35 31.7735) (end -3.884499 34.239001) (width 0.254) (layer B.Cu) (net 4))
 (segment (start -1.695251 34.239001) (end 3.140601 34.239001) (width 0.254) (layer B.Cu) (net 4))
 (segment (start -1.907017 34.239001) (end -1.695251 34.239001) (width 0.254) (layer B.Cu) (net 4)))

